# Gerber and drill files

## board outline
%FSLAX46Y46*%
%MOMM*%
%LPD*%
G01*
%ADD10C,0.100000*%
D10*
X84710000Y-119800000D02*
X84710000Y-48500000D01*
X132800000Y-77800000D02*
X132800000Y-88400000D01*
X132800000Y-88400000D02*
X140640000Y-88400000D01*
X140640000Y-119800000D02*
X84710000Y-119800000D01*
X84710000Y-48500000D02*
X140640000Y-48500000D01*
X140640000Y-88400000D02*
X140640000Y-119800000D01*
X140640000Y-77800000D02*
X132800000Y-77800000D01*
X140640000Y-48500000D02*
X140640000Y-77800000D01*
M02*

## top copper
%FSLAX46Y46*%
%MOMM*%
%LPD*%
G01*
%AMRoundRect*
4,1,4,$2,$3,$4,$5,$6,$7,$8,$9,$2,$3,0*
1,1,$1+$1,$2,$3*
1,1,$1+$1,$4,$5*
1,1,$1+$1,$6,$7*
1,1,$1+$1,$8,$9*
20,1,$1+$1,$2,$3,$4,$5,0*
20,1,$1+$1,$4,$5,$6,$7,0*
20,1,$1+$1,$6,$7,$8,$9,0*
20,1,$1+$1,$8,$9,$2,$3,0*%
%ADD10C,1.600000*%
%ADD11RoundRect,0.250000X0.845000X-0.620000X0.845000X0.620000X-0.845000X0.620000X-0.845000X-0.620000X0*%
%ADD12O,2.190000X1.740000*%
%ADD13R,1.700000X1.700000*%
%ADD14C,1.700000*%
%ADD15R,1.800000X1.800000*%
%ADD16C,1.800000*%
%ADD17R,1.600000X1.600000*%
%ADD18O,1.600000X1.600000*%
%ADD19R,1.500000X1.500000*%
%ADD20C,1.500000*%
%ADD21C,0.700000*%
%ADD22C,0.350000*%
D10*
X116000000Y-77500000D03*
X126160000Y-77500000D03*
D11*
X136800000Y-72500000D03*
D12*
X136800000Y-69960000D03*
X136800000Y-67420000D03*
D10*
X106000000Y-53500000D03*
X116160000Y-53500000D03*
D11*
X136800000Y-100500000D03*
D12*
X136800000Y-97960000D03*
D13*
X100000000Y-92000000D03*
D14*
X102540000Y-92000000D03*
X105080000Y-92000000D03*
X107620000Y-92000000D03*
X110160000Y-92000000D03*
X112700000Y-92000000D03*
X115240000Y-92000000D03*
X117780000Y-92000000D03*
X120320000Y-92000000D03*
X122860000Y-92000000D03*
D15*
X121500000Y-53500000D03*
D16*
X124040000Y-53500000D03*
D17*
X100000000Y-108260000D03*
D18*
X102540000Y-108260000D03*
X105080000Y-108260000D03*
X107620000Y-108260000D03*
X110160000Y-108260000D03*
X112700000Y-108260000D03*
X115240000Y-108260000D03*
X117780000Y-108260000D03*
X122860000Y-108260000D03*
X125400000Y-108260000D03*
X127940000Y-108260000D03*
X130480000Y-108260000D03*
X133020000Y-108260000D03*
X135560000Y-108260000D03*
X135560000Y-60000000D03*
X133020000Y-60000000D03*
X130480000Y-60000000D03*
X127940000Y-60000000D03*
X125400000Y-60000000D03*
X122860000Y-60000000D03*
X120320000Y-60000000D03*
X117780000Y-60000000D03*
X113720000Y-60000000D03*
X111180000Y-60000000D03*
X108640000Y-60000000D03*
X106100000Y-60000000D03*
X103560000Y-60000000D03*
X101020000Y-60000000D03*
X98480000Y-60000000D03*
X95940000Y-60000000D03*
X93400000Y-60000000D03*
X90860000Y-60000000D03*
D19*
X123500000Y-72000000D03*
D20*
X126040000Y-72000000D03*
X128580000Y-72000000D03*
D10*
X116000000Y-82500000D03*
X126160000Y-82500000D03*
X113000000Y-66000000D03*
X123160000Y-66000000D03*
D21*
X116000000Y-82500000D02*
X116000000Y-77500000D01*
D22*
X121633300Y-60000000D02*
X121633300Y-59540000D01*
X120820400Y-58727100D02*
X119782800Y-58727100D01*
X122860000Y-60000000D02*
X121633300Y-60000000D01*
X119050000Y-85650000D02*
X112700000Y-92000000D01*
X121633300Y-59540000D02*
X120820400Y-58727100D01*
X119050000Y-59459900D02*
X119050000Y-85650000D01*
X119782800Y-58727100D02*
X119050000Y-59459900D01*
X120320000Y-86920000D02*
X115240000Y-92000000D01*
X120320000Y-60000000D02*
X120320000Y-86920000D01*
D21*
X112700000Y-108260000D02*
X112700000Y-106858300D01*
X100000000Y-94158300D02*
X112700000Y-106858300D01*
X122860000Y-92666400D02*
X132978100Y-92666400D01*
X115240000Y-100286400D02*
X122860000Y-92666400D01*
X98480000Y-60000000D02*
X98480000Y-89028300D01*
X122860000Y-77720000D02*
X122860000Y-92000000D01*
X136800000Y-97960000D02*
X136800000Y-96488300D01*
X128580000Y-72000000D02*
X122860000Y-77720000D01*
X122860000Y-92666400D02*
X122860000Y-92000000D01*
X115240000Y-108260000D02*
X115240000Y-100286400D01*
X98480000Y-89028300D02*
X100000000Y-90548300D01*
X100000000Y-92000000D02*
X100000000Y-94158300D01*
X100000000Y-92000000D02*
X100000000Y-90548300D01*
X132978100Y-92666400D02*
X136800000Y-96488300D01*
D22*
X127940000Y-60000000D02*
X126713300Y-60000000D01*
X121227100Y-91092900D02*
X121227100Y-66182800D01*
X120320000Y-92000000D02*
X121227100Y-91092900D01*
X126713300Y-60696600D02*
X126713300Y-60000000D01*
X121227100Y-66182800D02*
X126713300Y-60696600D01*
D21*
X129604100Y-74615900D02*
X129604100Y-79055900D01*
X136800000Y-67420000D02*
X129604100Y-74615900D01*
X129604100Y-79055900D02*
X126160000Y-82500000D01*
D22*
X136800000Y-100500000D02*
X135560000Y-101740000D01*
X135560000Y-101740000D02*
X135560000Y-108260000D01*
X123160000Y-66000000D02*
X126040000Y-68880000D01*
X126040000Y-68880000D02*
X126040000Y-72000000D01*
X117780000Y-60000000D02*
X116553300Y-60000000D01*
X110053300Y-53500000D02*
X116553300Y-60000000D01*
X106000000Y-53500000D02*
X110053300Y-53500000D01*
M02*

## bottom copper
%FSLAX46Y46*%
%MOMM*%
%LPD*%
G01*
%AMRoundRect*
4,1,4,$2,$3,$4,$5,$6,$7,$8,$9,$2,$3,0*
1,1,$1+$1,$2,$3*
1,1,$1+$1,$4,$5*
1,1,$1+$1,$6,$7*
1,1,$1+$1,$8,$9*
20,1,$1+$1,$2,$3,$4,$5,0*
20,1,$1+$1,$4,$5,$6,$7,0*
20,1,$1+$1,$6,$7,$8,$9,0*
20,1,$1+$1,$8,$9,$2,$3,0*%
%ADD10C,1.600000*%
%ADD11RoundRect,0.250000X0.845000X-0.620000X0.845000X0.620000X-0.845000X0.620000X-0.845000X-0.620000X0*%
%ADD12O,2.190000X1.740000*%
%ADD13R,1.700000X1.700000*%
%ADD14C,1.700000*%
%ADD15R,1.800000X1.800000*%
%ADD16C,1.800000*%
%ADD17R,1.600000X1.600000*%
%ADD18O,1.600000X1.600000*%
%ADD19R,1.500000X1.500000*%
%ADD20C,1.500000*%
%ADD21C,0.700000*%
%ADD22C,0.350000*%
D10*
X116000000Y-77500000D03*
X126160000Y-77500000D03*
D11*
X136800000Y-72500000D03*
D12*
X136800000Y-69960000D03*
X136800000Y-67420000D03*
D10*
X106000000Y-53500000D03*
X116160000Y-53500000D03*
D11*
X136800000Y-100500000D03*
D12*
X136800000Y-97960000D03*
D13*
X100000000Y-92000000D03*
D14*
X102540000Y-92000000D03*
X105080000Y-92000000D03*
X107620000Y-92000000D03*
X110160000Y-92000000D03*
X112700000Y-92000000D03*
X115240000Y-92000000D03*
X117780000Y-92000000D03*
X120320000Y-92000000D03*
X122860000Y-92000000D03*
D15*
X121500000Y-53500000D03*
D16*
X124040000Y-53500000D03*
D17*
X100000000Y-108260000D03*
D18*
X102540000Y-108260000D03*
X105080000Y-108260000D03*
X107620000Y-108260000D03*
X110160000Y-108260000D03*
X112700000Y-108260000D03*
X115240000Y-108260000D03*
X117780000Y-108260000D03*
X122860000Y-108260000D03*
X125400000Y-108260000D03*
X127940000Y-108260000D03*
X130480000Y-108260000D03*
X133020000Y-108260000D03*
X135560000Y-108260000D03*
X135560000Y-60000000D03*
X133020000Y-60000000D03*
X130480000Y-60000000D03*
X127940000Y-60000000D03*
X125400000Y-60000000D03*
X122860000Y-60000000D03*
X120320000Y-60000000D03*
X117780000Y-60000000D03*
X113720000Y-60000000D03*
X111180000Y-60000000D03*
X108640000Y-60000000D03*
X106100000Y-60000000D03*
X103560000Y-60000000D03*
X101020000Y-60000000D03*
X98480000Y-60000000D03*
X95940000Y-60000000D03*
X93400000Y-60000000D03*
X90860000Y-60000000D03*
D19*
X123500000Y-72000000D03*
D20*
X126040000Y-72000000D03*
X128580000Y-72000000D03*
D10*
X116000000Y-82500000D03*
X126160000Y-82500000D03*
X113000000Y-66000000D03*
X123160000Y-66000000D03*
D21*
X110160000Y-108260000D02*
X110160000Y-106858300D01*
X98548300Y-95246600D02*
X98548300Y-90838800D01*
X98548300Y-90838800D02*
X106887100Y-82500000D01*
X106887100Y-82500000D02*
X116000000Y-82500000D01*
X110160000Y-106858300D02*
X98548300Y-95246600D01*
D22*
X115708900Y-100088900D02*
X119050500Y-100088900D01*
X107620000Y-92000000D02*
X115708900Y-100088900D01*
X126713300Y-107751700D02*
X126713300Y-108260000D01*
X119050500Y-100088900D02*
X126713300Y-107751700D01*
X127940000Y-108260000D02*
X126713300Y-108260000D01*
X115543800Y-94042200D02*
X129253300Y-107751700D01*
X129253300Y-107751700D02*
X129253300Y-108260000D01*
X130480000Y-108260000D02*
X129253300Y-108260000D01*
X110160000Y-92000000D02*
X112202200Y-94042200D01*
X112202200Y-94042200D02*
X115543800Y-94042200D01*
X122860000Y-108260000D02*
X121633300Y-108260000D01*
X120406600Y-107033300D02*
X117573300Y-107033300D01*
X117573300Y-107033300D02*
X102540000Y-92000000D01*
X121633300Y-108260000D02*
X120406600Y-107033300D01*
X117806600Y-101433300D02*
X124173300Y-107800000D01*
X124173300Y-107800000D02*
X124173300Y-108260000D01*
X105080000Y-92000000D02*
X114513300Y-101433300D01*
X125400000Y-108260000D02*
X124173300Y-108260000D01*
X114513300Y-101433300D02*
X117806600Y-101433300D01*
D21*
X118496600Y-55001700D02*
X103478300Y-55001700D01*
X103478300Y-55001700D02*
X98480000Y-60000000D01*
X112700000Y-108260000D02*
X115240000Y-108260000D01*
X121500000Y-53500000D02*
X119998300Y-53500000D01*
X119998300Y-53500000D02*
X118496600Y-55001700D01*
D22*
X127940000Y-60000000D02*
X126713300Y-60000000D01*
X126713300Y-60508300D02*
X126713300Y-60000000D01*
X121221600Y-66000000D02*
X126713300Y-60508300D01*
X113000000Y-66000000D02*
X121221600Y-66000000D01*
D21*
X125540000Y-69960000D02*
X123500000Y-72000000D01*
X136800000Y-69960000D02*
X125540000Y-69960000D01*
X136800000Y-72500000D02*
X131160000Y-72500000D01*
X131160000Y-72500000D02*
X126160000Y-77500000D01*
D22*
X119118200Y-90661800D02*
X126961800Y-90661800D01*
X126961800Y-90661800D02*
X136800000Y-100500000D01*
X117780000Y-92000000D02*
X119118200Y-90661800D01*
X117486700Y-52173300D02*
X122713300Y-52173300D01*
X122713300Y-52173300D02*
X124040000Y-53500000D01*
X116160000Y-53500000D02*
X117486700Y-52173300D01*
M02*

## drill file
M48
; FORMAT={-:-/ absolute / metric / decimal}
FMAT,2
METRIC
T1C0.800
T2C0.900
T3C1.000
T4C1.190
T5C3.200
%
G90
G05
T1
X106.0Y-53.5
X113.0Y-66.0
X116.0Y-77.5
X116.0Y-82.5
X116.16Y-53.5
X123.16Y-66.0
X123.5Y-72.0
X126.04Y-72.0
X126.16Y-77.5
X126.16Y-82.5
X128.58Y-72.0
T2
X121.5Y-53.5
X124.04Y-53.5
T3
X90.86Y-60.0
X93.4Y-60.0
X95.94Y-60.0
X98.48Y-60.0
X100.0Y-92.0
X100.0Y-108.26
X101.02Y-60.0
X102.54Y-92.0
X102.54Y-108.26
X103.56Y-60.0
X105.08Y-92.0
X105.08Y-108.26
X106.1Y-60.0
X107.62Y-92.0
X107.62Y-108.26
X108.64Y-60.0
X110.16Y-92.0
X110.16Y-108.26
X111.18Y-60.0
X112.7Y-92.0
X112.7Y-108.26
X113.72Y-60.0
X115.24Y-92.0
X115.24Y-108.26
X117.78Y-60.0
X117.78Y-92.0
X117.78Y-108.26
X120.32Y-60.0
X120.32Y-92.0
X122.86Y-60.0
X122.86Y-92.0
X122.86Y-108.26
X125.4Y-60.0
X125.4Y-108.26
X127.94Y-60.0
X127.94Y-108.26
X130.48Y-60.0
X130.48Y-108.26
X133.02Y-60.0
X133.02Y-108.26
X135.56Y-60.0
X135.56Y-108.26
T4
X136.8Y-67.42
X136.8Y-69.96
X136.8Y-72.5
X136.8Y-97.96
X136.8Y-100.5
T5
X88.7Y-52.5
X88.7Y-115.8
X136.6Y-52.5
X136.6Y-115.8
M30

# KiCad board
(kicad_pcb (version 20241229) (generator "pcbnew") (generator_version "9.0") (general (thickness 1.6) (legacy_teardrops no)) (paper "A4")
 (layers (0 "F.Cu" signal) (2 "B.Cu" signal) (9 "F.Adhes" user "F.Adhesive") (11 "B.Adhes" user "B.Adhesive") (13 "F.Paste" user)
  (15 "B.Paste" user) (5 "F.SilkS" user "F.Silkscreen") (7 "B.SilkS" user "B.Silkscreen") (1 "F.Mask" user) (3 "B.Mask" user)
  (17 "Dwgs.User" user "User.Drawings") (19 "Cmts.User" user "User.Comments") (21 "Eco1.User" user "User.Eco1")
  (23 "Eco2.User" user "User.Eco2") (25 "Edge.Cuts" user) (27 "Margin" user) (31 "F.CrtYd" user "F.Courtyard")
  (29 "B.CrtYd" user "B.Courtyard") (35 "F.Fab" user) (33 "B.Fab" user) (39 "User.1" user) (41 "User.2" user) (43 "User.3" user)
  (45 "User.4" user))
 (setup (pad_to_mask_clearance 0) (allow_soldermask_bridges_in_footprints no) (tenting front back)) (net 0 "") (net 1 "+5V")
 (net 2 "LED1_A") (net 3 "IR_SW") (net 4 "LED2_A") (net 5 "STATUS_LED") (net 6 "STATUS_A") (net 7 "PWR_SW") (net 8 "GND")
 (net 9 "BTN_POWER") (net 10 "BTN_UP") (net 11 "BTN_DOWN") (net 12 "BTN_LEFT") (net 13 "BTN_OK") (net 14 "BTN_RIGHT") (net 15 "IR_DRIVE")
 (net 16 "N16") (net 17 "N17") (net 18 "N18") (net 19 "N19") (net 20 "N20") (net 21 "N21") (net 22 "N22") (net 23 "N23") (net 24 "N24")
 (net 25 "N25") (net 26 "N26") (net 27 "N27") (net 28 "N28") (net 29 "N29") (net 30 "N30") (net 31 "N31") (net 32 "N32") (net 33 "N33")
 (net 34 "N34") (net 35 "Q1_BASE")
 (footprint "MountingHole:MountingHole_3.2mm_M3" (layer "F.Cu") (at 88.7 52.5)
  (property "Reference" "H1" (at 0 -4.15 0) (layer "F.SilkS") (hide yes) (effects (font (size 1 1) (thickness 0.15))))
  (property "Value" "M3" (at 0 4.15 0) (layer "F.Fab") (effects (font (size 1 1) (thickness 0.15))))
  (pad "" np_thru_hole circle (at 0 0) (size 3.2 3.2) (drill 3.2) (layers "*.Cu" "*.Mask")))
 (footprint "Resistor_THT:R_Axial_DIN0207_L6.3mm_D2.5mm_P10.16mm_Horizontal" (layer "F.Cu") (at 116 77.5)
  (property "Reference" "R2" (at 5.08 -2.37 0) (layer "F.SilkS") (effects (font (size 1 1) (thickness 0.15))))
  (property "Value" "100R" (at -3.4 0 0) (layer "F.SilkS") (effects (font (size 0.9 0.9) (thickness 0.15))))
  (pad "1" thru_hole circle (at 0 0) (size 1.6 1.6) (drill 0.8) (layers "*.Cu" "*.Mask") (remove_unused_layers no) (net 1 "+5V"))
  (pad "2" thru_hole circle (at 10.16 0) (size 1.6 1.6) (drill 0.8) (layers "*.Cu" "*.Mask") (remove_unused_layers no) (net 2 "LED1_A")))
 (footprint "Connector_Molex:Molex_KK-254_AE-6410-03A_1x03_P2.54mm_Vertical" (layer "F.Cu") (at 136.8 72.5 90)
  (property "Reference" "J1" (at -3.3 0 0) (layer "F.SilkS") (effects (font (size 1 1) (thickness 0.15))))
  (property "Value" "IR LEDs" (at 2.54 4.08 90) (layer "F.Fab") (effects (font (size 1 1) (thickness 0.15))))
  (pad "1" thru_hole roundrect (at 0 0 90) (size 1.74 2.19) (drill 1.19) (layers "*.Cu" "*.Mask") (remove_unused_layers no)
   (roundrect_rratio 0.143678) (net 2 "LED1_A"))
  (pad "2" thru_hole oval (at 2.54 0 90) (size 1.74 2.19) (drill 1.19) (layers "*.Cu" "*.Mask") (remove_unused_layers no) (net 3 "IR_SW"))
  (pad "3" thru_hole oval (at 5.08 0 90) (size 1.74 2.19) (drill 1.19) (layers "*.Cu" "*.Mask") (remove_unused_layers no) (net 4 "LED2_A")))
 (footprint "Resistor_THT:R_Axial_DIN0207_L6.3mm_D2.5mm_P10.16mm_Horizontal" (layer "F.Cu") (at 106 53.5)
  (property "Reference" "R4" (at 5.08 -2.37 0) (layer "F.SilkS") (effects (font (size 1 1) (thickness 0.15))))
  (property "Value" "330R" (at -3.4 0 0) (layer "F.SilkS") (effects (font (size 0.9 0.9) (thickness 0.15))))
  (pad "1" thru_hole circle (at 0 0) (size 1.6 1.6) (drill 0.8) (layers "*.Cu" "*.Mask") (remove_unused_layers no) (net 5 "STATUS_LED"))
  (pad "2" thru_hole circle (at 10.16 0) (size 1.6 1.6) (drill 0.8) (layers "*.Cu" "*.Mask") (remove_unused_layers no) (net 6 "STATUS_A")))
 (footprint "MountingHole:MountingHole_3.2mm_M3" (layer "F.Cu") (at 136.6 115.8)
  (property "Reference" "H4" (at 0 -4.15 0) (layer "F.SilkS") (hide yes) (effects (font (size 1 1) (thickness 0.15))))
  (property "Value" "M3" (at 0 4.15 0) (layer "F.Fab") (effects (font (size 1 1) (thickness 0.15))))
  (pad "" np_thru_hole circle (at 0 0) (size 3.2 3.2) (drill 3.2) (layers "*.Cu" "*.Mask")))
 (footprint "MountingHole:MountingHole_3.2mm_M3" (layer "F.Cu") (at 136.6 52.5)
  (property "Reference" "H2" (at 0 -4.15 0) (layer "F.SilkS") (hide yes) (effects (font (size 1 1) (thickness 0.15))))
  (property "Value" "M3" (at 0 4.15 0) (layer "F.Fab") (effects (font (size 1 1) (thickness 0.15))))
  (pad "" np_thru_hole circle (at 0 0) (size 3.2 3.2) (drill 3.2) (layers "*.Cu" "*.Mask")))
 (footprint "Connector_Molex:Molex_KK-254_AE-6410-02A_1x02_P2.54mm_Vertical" (layer "F.Cu") (at 136.8 100.5 90)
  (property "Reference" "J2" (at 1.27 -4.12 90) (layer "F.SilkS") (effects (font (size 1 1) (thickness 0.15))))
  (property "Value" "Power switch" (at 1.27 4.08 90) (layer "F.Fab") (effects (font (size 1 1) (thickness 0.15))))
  (pad "1" thru_hole roundrect (at 0 0 90) (size 1.74 2.19) (drill 1.19) (layers "*.Cu" "*.Mask") (remove_unused_layers no)
   (roundrect_rratio 0.143678) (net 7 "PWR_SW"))
  (pad "2" thru_hole oval (at 2.54 0 90) (size 1.74 2.19) (drill 1.19) (layers "*.Cu" "*.Mask") (remove_unused_layers no) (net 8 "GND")))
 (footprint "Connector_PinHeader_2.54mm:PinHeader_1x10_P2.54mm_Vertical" (layer "F.Cu") (at 100 92 90)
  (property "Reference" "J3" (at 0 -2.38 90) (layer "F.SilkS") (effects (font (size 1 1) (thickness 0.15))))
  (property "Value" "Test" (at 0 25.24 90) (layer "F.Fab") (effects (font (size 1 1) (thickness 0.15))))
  (pad "1" thru_hole rect (at 0 0 90) (size 1.7 1.7) (drill 1) (layers "*.Cu" "*.Mask") (remove_unused_layers no) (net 8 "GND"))
  (pad "2" thru_hole circle (at 0 2.54 90) (size 1.7 1.7) (drill 1) (layers "*.Cu" "*.Mask") (remove_unused_layers no) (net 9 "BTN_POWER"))
  (pad "3" thru_hole circle (at 0 5.08 90) (size 1.7 1.7) (drill 1) (layers "*.Cu" "*.Mask") (remove_unused_layers no) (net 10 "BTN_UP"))
  (pad "4" thru_hole circle (at 0 7.62 90) (size 1.7 1.7) (drill 1) (layers "*.Cu" "*.Mask") (remove_unused_layers no) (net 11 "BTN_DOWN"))
  (pad "5" thru_hole circle (at 0 10.16 90) (size 1.7 1.7) (drill 1) (layers "*.Cu" "*.Mask") (remove_unused_layers no) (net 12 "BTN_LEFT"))
  (pad "6" thru_hole circle (at 0 12.7 90) (size 1.7 1.7) (drill 1) (layers "*.Cu" "*.Mask") (remove_unused_layers no) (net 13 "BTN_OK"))
  (pad "7" thru_hole circle (at 0 15.24 90) (size 1.7 1.7) (drill 1) (layers "*.Cu" "*.Mask") (remove_unused_layers no) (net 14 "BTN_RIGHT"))
  (pad "8" thru_hole circle (at 0 17.78 90) (size 1.7 1.7) (drill 1) (layers "*.Cu" "*.Mask") (remove_unused_layers no) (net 7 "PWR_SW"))
  (pad "9" thru_hole circle (at 0 20.32 90) (size 1.7 1.7) (drill 1) (layers "*.Cu" "*.Mask") (remove_unused_layers no) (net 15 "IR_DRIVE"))
  (pad "10" thru_hole circle (at 0 22.86 90) (size 1.7 1.7) (drill 1) (layers "*.Cu" "*.Mask") (remove_unused_layers no) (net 8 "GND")))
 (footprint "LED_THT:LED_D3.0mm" (layer "F.Cu") (at 121.5 53.5)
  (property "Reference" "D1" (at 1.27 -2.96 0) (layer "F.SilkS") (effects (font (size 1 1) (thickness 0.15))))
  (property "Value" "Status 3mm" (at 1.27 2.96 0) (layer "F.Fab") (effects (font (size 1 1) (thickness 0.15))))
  (pad "1" thru_hole rect (at 0 0) (size 1.8 1.8) (drill 0.9) (layers "*.Cu" "*.Mask") (remove_unused_layers no) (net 8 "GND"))
  (pad "2" thru_hole circle (at 2.54 0) (size 1.8 1.8) (drill 0.9) (layers "*.Cu" "*.Mask") (remove_unused_layers no) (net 6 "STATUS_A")))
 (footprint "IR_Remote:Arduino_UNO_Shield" (layer "F.Cu") (at 100 60)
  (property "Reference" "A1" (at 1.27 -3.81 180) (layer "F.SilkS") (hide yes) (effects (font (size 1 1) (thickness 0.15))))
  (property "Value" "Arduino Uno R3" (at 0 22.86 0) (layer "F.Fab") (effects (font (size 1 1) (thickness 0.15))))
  (pad "1" thru_hole rect (at 0 48.26 90) (size 1.6 1.6) (drill 1) (layers "*.Cu" "*.Mask") (remove_unused_layers no) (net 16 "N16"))
  (pad "2" thru_hole oval (at 2.54 48.26 90) (size 1.6 1.6) (drill 1) (layers "*.Cu" "*.Mask") (remove_unused_layers no) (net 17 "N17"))
  (pad "3" thru_hole oval (at 5.08 48.26 90) (size 1.6 1.6) (drill 1) (layers "*.Cu" "*.Mask") (remove_unused_layers no) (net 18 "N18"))
  (pad "4" thru_hole oval (at 7.62 48.26 90) (size 1.6 1.6) (drill 1) (layers "*.Cu" "*.Mask") (remove_unused_layers no) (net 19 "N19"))
  (pad "5" thru_hole oval (at 10.16 48.26 90) (size 1.6 1.6) (drill 1) (layers "*.Cu" "*.Mask") (remove_unused_layers no) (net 1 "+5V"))
  (pad "6" thru_hole oval (at 12.7 48.26 90) (size 1.6 1.6) (drill 1) (layers "*.Cu" "*.Mask") (remove_unused_layers no) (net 8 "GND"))
  (pad "7" thru_hole oval (at 15.24 48.26 90) (size 1.6 1.6) (drill 1) (layers "*.Cu" "*.Mask") (remove_unused_layers no) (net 8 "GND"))
  (pad "8" thru_hole oval (at 17.78 48.26 90) (size 1.6 1.6) (drill 1) (layers "*.Cu" "*.Mask") (remove_unused_layers no) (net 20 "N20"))
  (pad "9" thru_hole oval (at 22.86 48.26 90) (size 1.6 1.6) (drill 1) (layers "*.Cu" "*.Mask") (remove_unused_layers no)
   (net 9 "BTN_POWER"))
  (pad "10" thru_hole oval (at 25.4 48.26 90) (size 1.6 1.6) (drill 1) (layers "*.Cu" "*.Mask") (remove_unused_layers no) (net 10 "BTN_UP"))
  (pad "11" thru_hole oval (at 27.94 48.26 90) (size 1.6 1.6) (drill 1) (layers "*.Cu" "*.Mask") (remove_unused_layers no)
   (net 11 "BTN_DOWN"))
  (pad "12" thru_hole oval (at 30.48 48.26 90) (size 1.6 1.6) (drill 1) (layers "*.Cu" "*.Mask") (remove_unused_layers no)
   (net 12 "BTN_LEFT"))
  (pad "13" thru_hole oval (at 33.02 48.26 90) (size 1.6 1.6) (drill 1) (layers "*.Cu" "*.Mask") (remove_unused_layers no) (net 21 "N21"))
  (pad "14" thru_hole oval (at 35.56 48.26 90) (size 1.6 1.6) (drill 1) (layers "*.Cu" "*.Mask") (remove_unused_layers no) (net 7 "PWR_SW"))
  (pad "15" thru_hole oval (at 35.56 0 90) (size 1.6 1.6) (drill 1) (layers "*.Cu" "*.Mask") (remove_unused_layers no) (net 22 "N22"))
  (pad "16" thru_hole oval (at 33.02 0 90) (size 1.6 1.6) (drill 1) (layers "*.Cu" "*.Mask") (remove_unused_layers no) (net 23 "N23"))
  (pad "17" thru_hole oval (at 30.48 0 90) (size 1.6 1.6) (drill 1) (layers "*.Cu" "*.Mask") (remove_unused_layers no) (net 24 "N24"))
  (pad "18" thru_hole oval (at 27.94 0 90) (size 1.6 1.6) (drill 1) (layers "*.Cu" "*.Mask") (remove_unused_layers no) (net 15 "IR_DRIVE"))
  (pad "19" thru_hole oval (at 25.4 0 90) (size 1.6 1.6) (drill 1) (layers "*.Cu" "*.Mask") (remove_unused_layers no) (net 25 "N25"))
  (pad "20" thru_hole oval (at 22.86 0 90) (size 1.6 1.6) (drill 1) (layers "*.Cu" "*.Mask") (remove_unused_layers no) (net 13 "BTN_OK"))
  (pad "21" thru_hole oval (at 20.32 0 90) (size 1.6 1.6) (drill 1) (layers "*.Cu" "*.Mask") (remove_unused_layers no) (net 14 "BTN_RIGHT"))
  (pad "22" thru_hole oval (at 17.78 0 90) (size 1.6 1.6) (drill 1) (layers "*.Cu" "*.Mask") (remove_unused_layers no) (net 5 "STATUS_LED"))
  (pad "23" thru_hole oval (at 13.72 0 90) (size 1.6 1.6) (drill 1) (layers "*.Cu" "*.Mask") (remove_unused_layers no) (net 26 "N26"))
  (pad "24" thru_hole oval (at 11.18 0 90) (size 1.6 1.6) (drill 1) (layers "*.Cu" "*.Mask") (remove_unused_layers no) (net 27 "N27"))
  (pad "25" thru_hole oval (at 8.64 0 90) (size 1.6 1.6) (drill 1) (layers "*.Cu" "*.Mask") (remove_unused_layers no) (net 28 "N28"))
  (pad "26" thru_hole oval (at 6.1 0 90) (size 1.6 1.6) (drill 1) (layers "*.Cu" "*.Mask") (remove_unused_layers no) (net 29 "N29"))
  (pad "27" thru_hole oval (at 3.56 0 90) (size 1.6 1.6) (drill 1) (layers "*.Cu" "*.Mask") (remove_unused_layers no) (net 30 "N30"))
  (pad "28" thru_hole oval (at 1.02 0 90) (size 1.6 1.6) (drill 1) (layers "*.Cu" "*.Mask") (remove_unused_layers no) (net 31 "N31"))
  (pad "29" thru_hole oval (at -1.52 0 90) (size 1.6 1.6) (drill 1) (layers "*.Cu" "*.Mask") (remove_unused_layers no) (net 8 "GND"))
  (pad "30" thru_hole oval (at -4.06 0 90) (size 1.6 1.6) (drill 1) (layers "*.Cu" "*.Mask") (remove_unused_layers no) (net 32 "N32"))
  (pad "31" thru_hole oval (at -6.6 0 90) (size 1.6 1.6) (drill 1) (layers "*.Cu" "*.Mask") (remove_unused_layers no) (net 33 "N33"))
  (pad "32" thru_hole oval (at -9.14 0 90) (size 1.6 1.6) (drill 1) (layers "*.Cu" "*.Mask") (remove_unused_layers no) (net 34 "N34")))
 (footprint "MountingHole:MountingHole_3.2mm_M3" (layer "F.Cu") (at 88.7 115.8)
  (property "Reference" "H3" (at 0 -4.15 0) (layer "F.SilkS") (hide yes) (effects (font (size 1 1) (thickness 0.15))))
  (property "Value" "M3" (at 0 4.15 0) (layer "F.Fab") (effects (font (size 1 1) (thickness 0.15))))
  (pad "" np_thru_hole circle (at 0 0) (size 3.2 3.2) (drill 3.2) (layers "*.Cu" "*.Mask")))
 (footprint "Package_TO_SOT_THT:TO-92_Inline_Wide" (layer "F.Cu") (at 123.5 72)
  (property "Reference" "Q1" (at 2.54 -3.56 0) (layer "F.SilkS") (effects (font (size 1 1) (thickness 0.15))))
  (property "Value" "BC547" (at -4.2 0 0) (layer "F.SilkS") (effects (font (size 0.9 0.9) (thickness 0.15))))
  (pad "1" thru_hole rect (at 0 0) (size 1.5 1.5) (drill 0.8) (layers "*.Cu" "*.Mask") (remove_unused_layers no) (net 3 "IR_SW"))
  (pad "2" thru_hole circle (at 2.54 0) (size 1.5 1.5) (drill 0.8) (layers "*.Cu" "*.Mask") (remove_unused_layers no) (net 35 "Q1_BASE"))
  (pad "3" thru_hole circle (at 5.08 0) (size 1.5 1.5) (drill 0.8) (layers "*.Cu" "*.Mask") (remove_unused_layers no) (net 8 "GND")))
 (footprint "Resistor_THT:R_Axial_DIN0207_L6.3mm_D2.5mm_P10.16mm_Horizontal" (layer "F.Cu") (at 116 82.5)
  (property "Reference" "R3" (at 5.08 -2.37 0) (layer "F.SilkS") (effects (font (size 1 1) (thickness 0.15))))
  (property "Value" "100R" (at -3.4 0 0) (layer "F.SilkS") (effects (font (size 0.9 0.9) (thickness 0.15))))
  (pad "1" thru_hole circle (at 0 0) (size 1.6 1.6) (drill 0.8) (layers "*.Cu" "*.Mask") (remove_unused_layers no) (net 1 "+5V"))
  (pad "2" thru_hole circle (at 10.16 0) (size 1.6 1.6) (drill 0.8) (layers "*.Cu" "*.Mask") (remove_unused_layers no) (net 4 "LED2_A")))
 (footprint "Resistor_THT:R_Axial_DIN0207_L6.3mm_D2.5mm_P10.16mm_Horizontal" (layer "F.Cu") (at 113 66)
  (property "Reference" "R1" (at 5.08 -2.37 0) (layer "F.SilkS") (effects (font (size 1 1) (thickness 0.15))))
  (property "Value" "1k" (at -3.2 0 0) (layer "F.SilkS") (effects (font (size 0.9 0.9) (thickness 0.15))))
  (pad "1" thru_hole circle (at 0 0) (size 1.6 1.6) (drill 0.8) (layers "*.Cu" "*.Mask") (remove_unused_layers no) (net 15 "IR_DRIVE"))
  (pad "2" thru_hole circle (at 10.16 0) (size 1.6 1.6) (drill 0.8) (layers "*.Cu" "*.Mask") (remove_unused_layers no) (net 35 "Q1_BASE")))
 (gr_line (start 84.71 119.8) (end 84.71 48.5) (stroke (width 0.1) (type default)) (layer "Edge.Cuts"))
 (gr_line (start 132.8 77.8) (end 132.8 88.4) (stroke (width 0.1) (type default)) (layer "Edge.Cuts"))
 (gr_line (start 132.8 88.4) (end 140.64 88.4) (stroke (width 0.1) (type default)) (layer "Edge.Cuts"))
 (gr_line (start 140.64 119.8) (end 84.71 119.8) (stroke (width 0.1) (type default)) (layer "Edge.Cuts"))
 (gr_line (start 84.71 48.5) (end 140.64 48.5) (stroke (width 0.1) (type default)) (layer "Edge.Cuts"))
 (gr_line (start 140.64 88.4) (end 140.64 119.8) (stroke (width 0.1) (type default)) (layer "Edge.Cuts"))
 (gr_line (start 140.64 77.8) (end 132.8 77.8) (stroke (width 0.1) (type default)) (layer "Edge.Cuts"))
 (gr_line (start 140.64 48.5) (end 140.64 77.8) (stroke (width 0.1) (type default)) (layer "Edge.Cuts"))
 (segment (start 116 82.5) (end 116 77.5) (width 0.7) (layer "F.Cu") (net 1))
 (segment (start 110.16 108.26) (end 110.16 106.8583) (width 0.7) (layer "B.Cu") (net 1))
 (segment (start 98.5483 95.2466) (end 98.5483 90.8388) (width 0.7) (layer "B.Cu") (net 1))
 (segment (start 98.5483 90.8388) (end 106.8871 82.5) (width 0.7) (layer "B.Cu") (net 1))
 (segment (start 106.8871 82.5) (end 116 82.5) (width 0.7) (layer "B.Cu") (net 1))
 (segment (start 110.16 106.8583) (end 98.5483 95.2466) (width 0.7) (layer "B.Cu") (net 1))
 (segment (start 115.7089 100.0889) (end 119.0505 100.0889) (width 0.35) (layer "B.Cu") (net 11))
 (segment (start 107.62 92) (end 115.7089 100.0889) (width 0.35) (layer "B.Cu") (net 11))
 (segment (start 126.7133 107.7517) (end 126.7133 108.26) (width 0.35) (layer "B.Cu") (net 11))
 (segment (start 119.0505 100.0889) (end 126.7133 107.7517) (width 0.35) (layer "B.Cu") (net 11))
 (segment (start 127.94 108.26) (end 126.7133 108.26) (width 0.35) (layer "B.Cu") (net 11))
 (segment (start 115.5438 94.0422) (end 129.2533 107.7517) (width 0.35) (layer "B.Cu") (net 12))
 (segment (start 129.2533 107.7517) (end 129.2533 108.26) (width 0.35) (layer "B.Cu") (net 12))
 (segment (start 130.48 108.26) (end 129.2533 108.26) (width 0.35) (layer "B.Cu") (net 12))
 (segment (start 110.16 92) (end 112.2022 94.0422) (width 0.35) (layer "B.Cu") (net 12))
 (segment (start 112.2022 94.0422) (end 115.5438 94.0422) (width 0.35) (layer "B.Cu") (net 12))
 (segment (start 121.6333 60) (end 121.6333 59.54) (width 0.35) (layer "F.Cu") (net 13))
 (segment (start 120.8204 58.7271) (end 119.7828 58.7271) (width 0.35) (layer "F.Cu") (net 13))
 (segment (start 122.86 60) (end 121.6333 60) (width 0.35) (layer "F.Cu") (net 13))
 (segment (start 119.05 85.65) (end 112.7 92) (width 0.35) (layer "F.Cu") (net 13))
 (segment (start 121.6333 59.54) (end 120.8204 58.7271) (width 0.35) (layer "F.Cu") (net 13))
 (segment (start 119.05 59.4599) (end 119.05 85.65) (width 0.35) (layer "F.Cu") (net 13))
 (segment (start 119.7828 58.7271) (end 119.05 59.4599) (width 0.35) (layer "F.Cu") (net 13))
 (segment (start 122.86 108.26) (end 121.6333 108.26) (width 0.35) (layer "B.Cu") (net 9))
 (segment (start 120.4066 107.0333) (end 117.5733 107.0333) (width 0.35) (layer "B.Cu") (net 9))
 (segment (start 117.5733 107.0333) (end 102.54 92) (width 0.35) (layer "B.Cu") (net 9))
 (segment (start 121.6333 108.26) (end 120.4066 107.0333) (width 0.35) (layer "B.Cu") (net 9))
 (segment (start 120.32 86.92) (end 115.24 92) (width 0.35) (layer "F.Cu") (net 14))
 (segment (start 120.32 60) (end 120.32 86.92) (width 0.35) (layer "F.Cu") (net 14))
 (segment (start 117.8066 101.4333) (end 124.1733 107.8) (width 0.35) (layer "B.Cu") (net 10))
 (segment (start 124.1733 107.8) (end 124.1733 108.26) (width 0.35) (layer "B.Cu") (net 10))
 (segment (start 105.08 92) (end 114.5133 101.4333) (width 0.35) (layer "B.Cu") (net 10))
 (segment (start 125.4 108.26) (end 124.1733 108.26) (width 0.35) (layer "B.Cu") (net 10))
 (segment (start 114.5133 101.4333) (end 117.8066 101.4333) (width 0.35) (layer "B.Cu") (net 10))
 (segment (start 112.7 108.26) (end 112.7 106.8583) (width 0.7) (layer "F.Cu") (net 8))
 (segment (start 100 94.1583) (end 112.7 106.8583) (width 0.7) (layer "F.Cu") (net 8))
 (segment (start 122.86 92.6664) (end 132.9781 92.6664) (width 0.7) (layer "F.Cu") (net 8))
 (segment (start 115.24 100.2864) (end 122.86 92.6664) (width 0.7) (layer "F.Cu") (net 8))
 (segment (start 98.48 60) (end 98.48 89.0283) (width 0.7) (layer "F.Cu") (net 8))
 (segment (start 122.86 77.72) (end 122.86 92) (width 0.7) (layer "F.Cu") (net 8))
 (segment (start 136.8 97.96) (end 136.8 96.4883) (width 0.7) (layer "F.Cu") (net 8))
 (segment (start 128.58 72) (end 122.86 77.72) (width 0.7) (layer "F.Cu") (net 8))
 (segment (start 122.86 92.6664) (end 122.86 92) (width 0.7) (layer "F.Cu") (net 8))
 (segment (start 115.24 108.26) (end 115.24 100.2864) (width 0.7) (layer "F.Cu") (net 8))
 (segment (start 98.48 89.0283) (end 100 90.5483) (width 0.7) (layer "F.Cu") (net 8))
 (segment (start 100 92) (end 100 94.1583) (width 0.7) (layer "F.Cu") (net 8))
 (segment (start 100 92) (end 100 90.5483) (width 0.7) (layer "F.Cu") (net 8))
 (segment (start 132.9781 92.6664) (end 136.8 96.4883) (width 0.7) (layer "F.Cu") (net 8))
 (segment (start 118.4966 55.0017) (end 103.4783 55.0017) (width 0.7) (layer "B.Cu") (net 8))
 (segment (start 103.4783 55.0017) (end 98.48 60) (width 0.7) (layer "B.Cu") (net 8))
 (segment (start 112.7 108.26) (end 115.24 108.26) (width 0.7) (layer "B.Cu") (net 8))
 (segment (start 121.5 53.5) (end 119.9983 53.5) (width 0.7) (layer "B.Cu") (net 8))
 (segment (start 119.9983 53.5) (end 118.4966 55.0017) (width 0.7) (layer "B.Cu") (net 8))
 (segment (start 127.94 60) (end 126.7133 60) (width 0.35) (layer "F.Cu") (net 15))
 (segment (start 121.2271 91.0929) (end 121.2271 66.1828) (width 0.35) (layer "F.Cu") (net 15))
 (segment (start 120.32 92) (end 121.2271 91.0929) (width 0.35) (layer "F.Cu") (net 15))
 (segment (start 126.7133 60.6966) (end 126.7133 60) (width 0.35) (layer "F.Cu") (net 15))
 (segment (start 121.2271 66.1828) (end 126.7133 60.6966) (width 0.35) (layer "F.Cu") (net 15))
 (segment (start 127.94 60) (end 126.7133 60) (width 0.35) (layer "B.Cu") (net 15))
 (segment (start 126.7133 60.5083) (end 126.7133 60) (width 0.35) (layer "B.Cu") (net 15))
 (segment (start 121.2216 66) (end 126.7133 60.5083) (width 0.35) (layer "B.Cu") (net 15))
 (segment (start 113 66) (end 121.2216 66) (width 0.35) (layer "B.Cu") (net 15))
 (segment (start 125.54 69.96) (end 123.5 72) (width 0.7) (layer "B.Cu") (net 3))
 (segment (start 136.8 69.96) (end 125.54 69.96) (width 0.7) (layer "B.Cu") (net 3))
 (segment (start 136.8 72.5) (end 131.16 72.5) (width 0.7) (layer "B.Cu") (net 2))
 (segment (start 131.16 72.5) (end 126.16 77.5) (width 0.7) (layer "B.Cu") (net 2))
 (segment (start 129.6041 74.6159) (end 129.6041 79.0559) (width 0.7) (layer "F.Cu") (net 4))
 (segment (start 136.8 67.42) (end 129.6041 74.6159) (width 0.7) (layer "F.Cu") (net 4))
 (segment (start 129.6041 79.0559) (end 126.16 82.5) (width 0.7) (layer "F.Cu") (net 4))
 (segment (start 136.8 100.5) (end 135.56 101.74) (width 0.35) (layer "F.Cu") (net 7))
 (segment (start 135.56 101.74) (end 135.56 108.26) (width 0.35) (layer "F.Cu") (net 7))
 (segment (start 119.1182 90.6618) (end 126.9618 90.6618) (width 0.35) (layer "B.Cu") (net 7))
 (segment (start 126.9618 90.6618) (end 136.8 100.5) (width 0.35) (layer "B.Cu") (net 7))
 (segment (start 117.78 92) (end 119.1182 90.6618) (width 0.35) (layer "B.Cu") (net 7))
 (segment (start 123.16 66) (end 126.04 68.88) (width 0.35) (layer "F.Cu") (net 35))
 (segment (start 126.04 68.88) (end 126.04 72) (width 0.35) (layer "F.Cu") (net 35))
 (segment (start 117.4867 52.1733) (end 122.7133 52.1733) (width 0.35) (layer "B.Cu") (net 6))
 (segment (start 122.7133 52.1733) (end 124.04 53.5) (width 0.35) (layer "B.Cu") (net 6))
 (segment (start 116.16 53.5) (end 117.4867 52.1733) (width 0.35) (layer "B.Cu") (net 6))
 (segment (start 117.78 60) (end 116.5533 60) (width 0.35) (layer "F.Cu") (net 5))
 (segment (start 110.0533 53.5) (end 116.5533 60) (width 0.35) (layer "F.Cu") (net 5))
 (segment (start 106 53.5) (end 110.0533 53.5) (width 0.35) (layer "F.Cu") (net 5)))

